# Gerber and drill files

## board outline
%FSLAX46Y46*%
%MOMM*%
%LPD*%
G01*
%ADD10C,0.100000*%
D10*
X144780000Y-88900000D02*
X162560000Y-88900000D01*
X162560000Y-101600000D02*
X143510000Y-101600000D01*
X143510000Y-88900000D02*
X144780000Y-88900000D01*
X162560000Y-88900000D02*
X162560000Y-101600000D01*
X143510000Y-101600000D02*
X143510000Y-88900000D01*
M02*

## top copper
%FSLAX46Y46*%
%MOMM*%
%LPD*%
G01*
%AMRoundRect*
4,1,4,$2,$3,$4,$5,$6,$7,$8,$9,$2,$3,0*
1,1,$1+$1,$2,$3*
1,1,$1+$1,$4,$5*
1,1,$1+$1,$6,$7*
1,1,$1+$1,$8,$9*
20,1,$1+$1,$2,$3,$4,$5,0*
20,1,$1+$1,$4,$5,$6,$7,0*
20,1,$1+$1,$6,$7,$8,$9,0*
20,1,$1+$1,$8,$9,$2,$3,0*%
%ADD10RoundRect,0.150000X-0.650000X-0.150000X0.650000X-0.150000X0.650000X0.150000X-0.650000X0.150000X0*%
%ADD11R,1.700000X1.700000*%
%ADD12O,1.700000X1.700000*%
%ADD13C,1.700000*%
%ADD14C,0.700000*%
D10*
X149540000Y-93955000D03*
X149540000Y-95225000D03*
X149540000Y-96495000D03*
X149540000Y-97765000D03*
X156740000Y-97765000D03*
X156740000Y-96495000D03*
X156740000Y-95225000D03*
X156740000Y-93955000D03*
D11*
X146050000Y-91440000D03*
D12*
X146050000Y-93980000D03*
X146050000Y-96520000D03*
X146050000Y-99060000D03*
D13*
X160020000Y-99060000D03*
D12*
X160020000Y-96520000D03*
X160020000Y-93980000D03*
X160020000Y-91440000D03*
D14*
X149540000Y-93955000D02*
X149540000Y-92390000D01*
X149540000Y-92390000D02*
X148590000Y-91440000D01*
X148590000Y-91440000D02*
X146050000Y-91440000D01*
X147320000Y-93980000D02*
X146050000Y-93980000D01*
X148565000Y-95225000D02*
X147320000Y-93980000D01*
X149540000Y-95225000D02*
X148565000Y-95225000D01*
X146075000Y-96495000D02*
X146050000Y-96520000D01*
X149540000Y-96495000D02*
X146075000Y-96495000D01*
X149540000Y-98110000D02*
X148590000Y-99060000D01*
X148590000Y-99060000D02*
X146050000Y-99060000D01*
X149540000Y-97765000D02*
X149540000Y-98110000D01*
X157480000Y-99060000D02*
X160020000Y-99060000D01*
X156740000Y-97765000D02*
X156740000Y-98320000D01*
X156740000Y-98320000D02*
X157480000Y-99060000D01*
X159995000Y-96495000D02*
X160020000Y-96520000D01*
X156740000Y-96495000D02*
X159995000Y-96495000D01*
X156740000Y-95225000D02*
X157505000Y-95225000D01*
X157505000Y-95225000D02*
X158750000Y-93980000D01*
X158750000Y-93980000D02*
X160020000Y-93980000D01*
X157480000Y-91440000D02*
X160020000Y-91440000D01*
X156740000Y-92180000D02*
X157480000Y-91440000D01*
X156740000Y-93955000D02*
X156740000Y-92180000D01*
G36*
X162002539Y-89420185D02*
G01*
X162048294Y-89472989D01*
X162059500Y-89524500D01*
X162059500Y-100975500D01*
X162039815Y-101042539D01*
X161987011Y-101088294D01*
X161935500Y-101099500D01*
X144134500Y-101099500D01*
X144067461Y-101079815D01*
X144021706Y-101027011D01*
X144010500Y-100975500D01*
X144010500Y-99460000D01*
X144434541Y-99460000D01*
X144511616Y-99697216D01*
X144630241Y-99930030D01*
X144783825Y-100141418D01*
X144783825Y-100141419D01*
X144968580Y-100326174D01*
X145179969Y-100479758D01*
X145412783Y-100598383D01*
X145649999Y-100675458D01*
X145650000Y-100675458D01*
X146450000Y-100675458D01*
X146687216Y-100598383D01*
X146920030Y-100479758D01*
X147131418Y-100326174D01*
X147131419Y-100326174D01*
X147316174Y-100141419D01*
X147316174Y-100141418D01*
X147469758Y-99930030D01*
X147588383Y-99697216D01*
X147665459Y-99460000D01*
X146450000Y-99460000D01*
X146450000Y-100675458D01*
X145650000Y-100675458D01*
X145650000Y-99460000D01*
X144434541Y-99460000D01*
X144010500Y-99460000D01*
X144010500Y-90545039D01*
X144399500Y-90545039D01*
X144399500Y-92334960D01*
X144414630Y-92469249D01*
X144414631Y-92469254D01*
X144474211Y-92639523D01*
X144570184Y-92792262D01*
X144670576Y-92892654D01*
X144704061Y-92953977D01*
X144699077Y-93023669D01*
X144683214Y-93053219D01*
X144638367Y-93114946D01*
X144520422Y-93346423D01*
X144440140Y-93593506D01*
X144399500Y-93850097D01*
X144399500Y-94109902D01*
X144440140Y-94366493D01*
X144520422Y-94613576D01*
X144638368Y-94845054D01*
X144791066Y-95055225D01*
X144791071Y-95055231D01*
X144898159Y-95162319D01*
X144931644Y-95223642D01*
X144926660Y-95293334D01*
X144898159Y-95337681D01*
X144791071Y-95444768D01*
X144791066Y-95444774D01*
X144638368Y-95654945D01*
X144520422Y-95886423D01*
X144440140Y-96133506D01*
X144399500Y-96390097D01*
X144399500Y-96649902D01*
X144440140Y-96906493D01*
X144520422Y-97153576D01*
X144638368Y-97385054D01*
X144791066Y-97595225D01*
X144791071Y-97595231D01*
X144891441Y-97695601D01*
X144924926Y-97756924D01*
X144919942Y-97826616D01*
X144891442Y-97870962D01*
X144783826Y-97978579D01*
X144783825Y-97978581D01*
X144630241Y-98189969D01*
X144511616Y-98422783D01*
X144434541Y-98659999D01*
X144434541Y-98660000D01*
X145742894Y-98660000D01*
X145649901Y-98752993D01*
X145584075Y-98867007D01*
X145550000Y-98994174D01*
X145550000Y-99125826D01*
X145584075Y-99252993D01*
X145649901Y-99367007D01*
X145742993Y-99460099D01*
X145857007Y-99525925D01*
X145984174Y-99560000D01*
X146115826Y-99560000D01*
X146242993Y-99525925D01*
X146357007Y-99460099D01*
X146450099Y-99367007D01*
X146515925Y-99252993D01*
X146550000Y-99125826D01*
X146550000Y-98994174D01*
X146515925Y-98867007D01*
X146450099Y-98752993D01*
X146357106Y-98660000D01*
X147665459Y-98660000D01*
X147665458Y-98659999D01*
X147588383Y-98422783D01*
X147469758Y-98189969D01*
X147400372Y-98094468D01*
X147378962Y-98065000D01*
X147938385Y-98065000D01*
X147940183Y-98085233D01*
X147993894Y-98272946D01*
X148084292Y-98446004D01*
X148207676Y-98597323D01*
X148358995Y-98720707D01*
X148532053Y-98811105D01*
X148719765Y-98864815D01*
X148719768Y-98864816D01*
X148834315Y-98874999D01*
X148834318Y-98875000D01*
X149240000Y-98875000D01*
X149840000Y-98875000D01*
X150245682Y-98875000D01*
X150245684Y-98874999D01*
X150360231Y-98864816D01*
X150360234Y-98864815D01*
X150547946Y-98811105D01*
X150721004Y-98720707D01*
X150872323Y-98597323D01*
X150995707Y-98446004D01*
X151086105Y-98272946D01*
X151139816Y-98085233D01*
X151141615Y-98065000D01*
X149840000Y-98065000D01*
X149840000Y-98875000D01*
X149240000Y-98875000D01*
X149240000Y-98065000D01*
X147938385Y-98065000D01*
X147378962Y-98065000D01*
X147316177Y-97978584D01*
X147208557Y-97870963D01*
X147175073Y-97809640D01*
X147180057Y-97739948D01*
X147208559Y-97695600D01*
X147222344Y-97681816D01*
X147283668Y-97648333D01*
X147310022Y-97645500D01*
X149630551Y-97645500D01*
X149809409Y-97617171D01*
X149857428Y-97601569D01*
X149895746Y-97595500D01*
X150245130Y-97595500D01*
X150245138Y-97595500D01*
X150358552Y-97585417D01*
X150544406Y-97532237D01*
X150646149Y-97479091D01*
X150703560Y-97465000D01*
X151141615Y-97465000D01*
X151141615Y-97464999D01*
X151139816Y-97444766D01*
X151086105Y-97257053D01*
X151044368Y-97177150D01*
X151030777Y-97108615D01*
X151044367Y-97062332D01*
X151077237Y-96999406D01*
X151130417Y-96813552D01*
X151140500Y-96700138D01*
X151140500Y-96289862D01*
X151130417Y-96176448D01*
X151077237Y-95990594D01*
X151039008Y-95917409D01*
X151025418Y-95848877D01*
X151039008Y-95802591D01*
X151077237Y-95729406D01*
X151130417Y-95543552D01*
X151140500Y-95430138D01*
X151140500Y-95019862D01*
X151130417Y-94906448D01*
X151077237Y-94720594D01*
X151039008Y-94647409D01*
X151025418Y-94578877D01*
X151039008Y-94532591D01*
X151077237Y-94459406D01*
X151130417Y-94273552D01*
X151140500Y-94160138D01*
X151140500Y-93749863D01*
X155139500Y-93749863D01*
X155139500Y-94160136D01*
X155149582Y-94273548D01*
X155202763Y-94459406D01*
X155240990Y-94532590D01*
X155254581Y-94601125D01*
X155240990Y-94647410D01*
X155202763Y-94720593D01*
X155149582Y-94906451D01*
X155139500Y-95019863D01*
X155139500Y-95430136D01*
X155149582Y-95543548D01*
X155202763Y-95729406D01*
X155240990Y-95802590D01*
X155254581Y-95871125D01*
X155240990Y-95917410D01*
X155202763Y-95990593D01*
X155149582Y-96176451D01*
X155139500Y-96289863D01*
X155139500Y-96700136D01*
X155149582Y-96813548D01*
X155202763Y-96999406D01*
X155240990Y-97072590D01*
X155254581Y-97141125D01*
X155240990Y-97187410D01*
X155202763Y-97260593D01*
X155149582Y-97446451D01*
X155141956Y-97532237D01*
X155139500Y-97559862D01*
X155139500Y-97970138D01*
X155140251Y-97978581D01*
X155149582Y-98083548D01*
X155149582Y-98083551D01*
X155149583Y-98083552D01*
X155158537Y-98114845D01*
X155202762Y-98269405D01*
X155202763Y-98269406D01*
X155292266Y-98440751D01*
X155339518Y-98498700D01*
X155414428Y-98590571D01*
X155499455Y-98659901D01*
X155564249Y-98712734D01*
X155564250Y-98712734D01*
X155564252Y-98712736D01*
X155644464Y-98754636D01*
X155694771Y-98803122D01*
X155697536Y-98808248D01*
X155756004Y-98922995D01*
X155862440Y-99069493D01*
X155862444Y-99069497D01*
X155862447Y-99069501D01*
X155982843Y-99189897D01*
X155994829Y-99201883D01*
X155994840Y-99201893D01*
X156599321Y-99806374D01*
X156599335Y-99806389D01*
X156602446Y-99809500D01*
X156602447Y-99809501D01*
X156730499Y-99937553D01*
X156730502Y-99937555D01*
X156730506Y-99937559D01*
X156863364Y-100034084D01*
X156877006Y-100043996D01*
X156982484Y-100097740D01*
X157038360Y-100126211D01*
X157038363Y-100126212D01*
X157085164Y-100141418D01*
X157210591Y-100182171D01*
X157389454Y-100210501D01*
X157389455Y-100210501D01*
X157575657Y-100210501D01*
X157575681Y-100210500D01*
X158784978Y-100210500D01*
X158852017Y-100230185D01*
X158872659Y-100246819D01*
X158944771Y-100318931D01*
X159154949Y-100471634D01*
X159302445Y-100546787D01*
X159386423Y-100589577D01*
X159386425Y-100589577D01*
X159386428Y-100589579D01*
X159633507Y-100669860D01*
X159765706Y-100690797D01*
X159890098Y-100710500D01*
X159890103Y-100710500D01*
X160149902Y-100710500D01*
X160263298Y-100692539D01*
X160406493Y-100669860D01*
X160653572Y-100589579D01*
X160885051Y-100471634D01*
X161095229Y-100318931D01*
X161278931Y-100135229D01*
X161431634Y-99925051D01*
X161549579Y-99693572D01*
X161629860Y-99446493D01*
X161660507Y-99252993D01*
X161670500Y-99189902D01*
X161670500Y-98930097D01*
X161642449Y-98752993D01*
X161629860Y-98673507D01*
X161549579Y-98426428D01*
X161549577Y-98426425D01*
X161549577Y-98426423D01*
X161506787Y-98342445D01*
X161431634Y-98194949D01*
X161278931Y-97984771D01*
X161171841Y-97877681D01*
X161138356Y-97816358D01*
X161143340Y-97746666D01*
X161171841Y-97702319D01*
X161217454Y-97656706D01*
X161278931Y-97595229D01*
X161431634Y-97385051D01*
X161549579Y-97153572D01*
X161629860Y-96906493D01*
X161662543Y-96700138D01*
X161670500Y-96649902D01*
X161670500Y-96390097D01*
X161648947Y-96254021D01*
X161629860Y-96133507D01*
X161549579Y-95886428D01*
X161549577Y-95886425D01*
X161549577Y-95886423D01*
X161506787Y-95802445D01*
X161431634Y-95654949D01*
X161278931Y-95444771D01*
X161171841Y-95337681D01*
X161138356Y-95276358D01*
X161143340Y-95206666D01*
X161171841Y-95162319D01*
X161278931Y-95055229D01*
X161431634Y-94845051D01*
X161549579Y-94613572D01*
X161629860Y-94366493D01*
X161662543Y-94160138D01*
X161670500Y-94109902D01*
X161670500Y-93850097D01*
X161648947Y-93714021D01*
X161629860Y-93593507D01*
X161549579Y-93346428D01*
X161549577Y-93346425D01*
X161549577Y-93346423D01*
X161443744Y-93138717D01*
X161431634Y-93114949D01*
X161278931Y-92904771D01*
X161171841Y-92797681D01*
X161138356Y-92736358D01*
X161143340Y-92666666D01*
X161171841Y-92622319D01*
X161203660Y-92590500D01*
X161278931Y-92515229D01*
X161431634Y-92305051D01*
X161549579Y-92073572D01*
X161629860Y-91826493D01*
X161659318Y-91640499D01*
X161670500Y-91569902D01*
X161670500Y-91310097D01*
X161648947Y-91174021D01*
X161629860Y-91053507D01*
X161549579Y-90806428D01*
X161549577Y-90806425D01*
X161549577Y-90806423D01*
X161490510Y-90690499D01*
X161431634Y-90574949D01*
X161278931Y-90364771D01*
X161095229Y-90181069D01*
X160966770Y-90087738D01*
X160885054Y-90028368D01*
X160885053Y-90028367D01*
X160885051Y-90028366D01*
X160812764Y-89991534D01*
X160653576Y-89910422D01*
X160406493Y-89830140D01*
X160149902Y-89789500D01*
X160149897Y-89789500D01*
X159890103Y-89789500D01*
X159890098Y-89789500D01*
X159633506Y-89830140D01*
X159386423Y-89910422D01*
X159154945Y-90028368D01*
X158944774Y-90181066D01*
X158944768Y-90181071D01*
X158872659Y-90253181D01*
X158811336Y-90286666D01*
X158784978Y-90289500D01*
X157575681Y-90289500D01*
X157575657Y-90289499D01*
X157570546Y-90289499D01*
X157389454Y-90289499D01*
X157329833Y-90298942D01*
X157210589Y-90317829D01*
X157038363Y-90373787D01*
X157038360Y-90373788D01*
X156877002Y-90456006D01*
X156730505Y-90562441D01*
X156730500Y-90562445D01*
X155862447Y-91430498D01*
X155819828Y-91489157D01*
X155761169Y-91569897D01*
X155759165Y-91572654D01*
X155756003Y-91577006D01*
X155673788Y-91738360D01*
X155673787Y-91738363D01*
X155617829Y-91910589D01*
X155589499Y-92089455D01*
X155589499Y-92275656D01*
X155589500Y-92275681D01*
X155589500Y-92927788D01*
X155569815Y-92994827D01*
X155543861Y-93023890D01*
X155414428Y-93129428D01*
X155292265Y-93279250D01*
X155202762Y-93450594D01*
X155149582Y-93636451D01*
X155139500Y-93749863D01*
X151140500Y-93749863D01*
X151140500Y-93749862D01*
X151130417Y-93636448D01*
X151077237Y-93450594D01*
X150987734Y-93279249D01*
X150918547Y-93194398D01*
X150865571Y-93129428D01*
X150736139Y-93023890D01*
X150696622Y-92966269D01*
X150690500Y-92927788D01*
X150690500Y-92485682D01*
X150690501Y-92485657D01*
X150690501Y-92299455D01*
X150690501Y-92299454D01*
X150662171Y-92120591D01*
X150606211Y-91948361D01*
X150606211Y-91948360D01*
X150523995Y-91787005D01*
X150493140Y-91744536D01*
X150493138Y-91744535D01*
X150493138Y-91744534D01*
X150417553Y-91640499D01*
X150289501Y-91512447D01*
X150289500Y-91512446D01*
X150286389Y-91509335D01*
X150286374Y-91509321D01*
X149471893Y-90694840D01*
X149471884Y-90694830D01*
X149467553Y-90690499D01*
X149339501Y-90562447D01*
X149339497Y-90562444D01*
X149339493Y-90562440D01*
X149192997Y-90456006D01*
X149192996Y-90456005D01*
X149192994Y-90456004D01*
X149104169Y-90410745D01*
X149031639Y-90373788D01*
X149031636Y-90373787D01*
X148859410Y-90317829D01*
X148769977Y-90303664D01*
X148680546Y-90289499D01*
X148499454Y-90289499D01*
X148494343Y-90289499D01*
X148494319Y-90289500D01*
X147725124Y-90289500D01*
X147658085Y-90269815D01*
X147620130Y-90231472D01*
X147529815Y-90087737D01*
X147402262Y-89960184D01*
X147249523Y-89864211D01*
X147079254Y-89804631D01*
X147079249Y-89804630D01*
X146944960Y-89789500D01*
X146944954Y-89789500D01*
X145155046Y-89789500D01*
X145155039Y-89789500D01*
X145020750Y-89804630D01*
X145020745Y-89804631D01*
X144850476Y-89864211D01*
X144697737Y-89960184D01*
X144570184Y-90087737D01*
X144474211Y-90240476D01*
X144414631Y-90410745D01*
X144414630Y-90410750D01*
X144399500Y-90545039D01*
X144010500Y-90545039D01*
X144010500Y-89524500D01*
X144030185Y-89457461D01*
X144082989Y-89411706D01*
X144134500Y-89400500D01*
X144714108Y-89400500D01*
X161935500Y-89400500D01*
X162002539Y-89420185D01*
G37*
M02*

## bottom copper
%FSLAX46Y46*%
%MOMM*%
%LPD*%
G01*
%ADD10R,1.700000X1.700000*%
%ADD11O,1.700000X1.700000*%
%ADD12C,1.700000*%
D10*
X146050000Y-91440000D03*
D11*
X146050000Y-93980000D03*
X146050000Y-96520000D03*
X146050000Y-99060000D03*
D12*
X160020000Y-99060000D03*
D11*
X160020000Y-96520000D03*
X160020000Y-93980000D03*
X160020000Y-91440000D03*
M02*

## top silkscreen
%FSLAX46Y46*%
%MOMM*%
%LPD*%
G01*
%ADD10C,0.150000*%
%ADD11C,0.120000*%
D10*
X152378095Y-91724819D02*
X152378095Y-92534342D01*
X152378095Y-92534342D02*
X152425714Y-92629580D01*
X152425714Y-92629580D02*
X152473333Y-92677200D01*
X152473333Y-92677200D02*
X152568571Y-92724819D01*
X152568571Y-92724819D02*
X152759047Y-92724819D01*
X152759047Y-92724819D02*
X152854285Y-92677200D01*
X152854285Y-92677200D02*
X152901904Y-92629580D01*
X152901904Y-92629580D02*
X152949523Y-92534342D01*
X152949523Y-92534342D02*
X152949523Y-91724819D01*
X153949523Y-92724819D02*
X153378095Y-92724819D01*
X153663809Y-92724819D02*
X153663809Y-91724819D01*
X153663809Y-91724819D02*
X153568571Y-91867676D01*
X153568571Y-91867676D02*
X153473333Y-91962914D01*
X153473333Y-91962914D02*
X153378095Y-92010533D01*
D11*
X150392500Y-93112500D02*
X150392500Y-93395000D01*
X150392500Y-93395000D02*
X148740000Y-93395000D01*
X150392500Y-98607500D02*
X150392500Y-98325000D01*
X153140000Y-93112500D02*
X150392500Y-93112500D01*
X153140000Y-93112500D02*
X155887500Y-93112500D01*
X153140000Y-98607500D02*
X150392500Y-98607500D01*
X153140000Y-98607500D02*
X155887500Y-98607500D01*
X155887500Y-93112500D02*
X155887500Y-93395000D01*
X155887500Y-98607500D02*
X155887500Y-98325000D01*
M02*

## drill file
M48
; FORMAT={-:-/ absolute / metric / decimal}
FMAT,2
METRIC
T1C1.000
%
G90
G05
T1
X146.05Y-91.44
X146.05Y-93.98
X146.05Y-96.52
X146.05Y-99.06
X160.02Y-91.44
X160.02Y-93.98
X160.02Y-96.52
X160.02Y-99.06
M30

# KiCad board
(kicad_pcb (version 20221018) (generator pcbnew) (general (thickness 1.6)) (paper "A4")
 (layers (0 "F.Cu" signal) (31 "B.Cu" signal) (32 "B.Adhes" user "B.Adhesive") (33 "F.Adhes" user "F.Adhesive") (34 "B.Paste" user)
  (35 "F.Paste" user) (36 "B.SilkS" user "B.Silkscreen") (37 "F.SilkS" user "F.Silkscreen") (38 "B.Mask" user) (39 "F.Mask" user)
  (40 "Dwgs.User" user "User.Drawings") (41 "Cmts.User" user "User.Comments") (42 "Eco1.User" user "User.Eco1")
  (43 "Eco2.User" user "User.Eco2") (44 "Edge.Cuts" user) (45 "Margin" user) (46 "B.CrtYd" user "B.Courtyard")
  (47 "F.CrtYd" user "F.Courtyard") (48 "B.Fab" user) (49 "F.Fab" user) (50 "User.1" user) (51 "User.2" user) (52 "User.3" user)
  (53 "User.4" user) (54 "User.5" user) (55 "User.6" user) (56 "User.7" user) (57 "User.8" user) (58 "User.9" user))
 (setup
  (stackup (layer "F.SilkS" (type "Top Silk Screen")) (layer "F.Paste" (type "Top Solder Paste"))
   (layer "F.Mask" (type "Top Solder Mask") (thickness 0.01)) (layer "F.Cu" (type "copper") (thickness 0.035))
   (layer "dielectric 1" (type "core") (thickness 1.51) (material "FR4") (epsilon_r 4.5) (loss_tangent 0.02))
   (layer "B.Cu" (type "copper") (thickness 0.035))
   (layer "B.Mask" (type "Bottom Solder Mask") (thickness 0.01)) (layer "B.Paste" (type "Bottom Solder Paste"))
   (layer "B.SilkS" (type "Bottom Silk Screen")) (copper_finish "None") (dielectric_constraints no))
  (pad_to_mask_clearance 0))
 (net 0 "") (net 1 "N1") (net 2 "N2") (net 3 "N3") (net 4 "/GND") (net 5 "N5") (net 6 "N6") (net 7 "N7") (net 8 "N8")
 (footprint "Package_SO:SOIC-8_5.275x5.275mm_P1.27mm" (layer "F.Cu") (at 153.14 95.86)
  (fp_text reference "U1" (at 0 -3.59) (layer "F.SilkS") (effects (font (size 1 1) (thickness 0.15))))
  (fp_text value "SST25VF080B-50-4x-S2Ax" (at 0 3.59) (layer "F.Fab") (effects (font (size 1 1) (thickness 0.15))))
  (fp_line (start -2.7475 -2.7475) (end -2.7475 -2.465) (stroke (width 0.12) (type solid)) (layer "F.SilkS"))
  (fp_line (start -2.7475 -2.465) (end -4.4 -2.465) (stroke (width 0.12) (type solid)) (layer "F.SilkS"))
  (fp_line (start -2.7475 2.7475) (end -2.7475 2.465) (stroke (width 0.12) (type solid)) (layer "F.SilkS"))
  (fp_line (start 0 -2.7475) (end -2.7475 -2.7475) (stroke (width 0.12) (type solid)) (layer "F.SilkS"))
  (fp_line (start 0 -2.7475) (end 2.7475 -2.7475) (stroke (width 0.12) (type solid)) (layer "F.SilkS"))
  (fp_line (start 0 2.7475) (end -2.7475 2.7475) (stroke (width 0.12) (type solid)) (layer "F.SilkS"))
  (fp_line (start 0 2.7475) (end 2.7475 2.7475) (stroke (width 0.12) (type solid)) (layer "F.SilkS"))
  (fp_line (start 2.7475 -2.7475) (end 2.7475 -2.465) (stroke (width 0.12) (type solid)) (layer "F.SilkS"))
  (fp_line (start 2.7475 2.7475) (end 2.7475 2.465) (stroke (width 0.12) (type solid)) (layer "F.SilkS"))
  (pad "1" smd roundrect (at -3.6 -1.905) (size 1.6 0.6) (layers "F.Cu" "F.Paste" "F.Mask") (roundrect_rratio 0.25) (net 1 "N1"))
  (pad "2" smd roundrect (at -3.6 -0.635) (size 1.6 0.6) (layers "F.Cu" "F.Paste" "F.Mask") (roundrect_rratio 0.25) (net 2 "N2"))
  (pad "3" smd roundrect (at -3.6 0.635) (size 1.6 0.6) (layers "F.Cu" "F.Paste" "F.Mask") (roundrect_rratio 0.25) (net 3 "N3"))
  (pad "4" smd roundrect (at -3.6 1.905) (size 1.6 0.6) (layers "F.Cu" "F.Paste" "F.Mask") (roundrect_rratio 0.25) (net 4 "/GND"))
  (pad "5" smd roundrect (at 3.6 1.905) (size 1.6 0.6) (layers "F.Cu" "F.Paste" "F.Mask") (roundrect_rratio 0.25) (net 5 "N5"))
  (pad "6" smd roundrect (at 3.6 0.635) (size 1.6 0.6) (layers "F.Cu" "F.Paste" "F.Mask") (roundrect_rratio 0.25) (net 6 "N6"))
  (pad "7" smd roundrect (at 3.6 -0.635) (size 1.6 0.6) (layers "F.Cu" "F.Paste" "F.Mask") (roundrect_rratio 0.25) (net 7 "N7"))
  (pad "8" smd roundrect (at 3.6 -1.905) (size 1.6 0.6) (layers "F.Cu" "F.Paste" "F.Mask") (roundrect_rratio 0.25) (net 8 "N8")))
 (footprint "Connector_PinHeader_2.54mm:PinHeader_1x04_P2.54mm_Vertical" (layer "B.Cu") (at 146.05 91.44 180)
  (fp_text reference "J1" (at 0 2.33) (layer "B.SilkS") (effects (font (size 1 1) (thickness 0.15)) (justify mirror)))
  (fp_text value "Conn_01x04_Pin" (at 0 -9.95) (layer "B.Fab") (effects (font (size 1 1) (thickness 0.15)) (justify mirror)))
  (pad "1" thru_hole rect (at 0 0 180) (size 1.7 1.7) (drill 1) (layers "*.Cu" "*.Mask") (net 1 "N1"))
  (pad "2" thru_hole oval (at 0 -2.54 180) (size 1.7 1.7) (drill 1) (layers "*.Cu" "*.Mask") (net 2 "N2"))
  (pad "3" thru_hole oval (at 0 -5.08 180) (size 1.7 1.7) (drill 1) (layers "*.Cu" "*.Mask") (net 3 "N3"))
  (pad "4" thru_hole oval (at 0 -7.62 180) (size 1.7 1.7) (drill 1) (layers "*.Cu" "*.Mask") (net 4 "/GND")))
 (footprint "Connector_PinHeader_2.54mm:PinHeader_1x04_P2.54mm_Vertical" (layer "B.Cu") (at 160.02 99.06)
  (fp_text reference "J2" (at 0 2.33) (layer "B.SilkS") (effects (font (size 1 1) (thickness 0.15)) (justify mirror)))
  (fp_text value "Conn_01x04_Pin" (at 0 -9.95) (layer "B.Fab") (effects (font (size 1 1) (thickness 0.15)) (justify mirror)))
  (pad "5" thru_hole circle (at 0 0) (size 1.7 1.7) (drill 1) (layers "*.Cu" "*.Mask") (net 5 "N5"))
  (pad "6" thru_hole oval (at 0 -2.54) (size 1.7 1.7) (drill 1) (layers "*.Cu" "*.Mask") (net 6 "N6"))
  (pad "7" thru_hole oval (at 0 -5.08) (size 1.7 1.7) (drill 1) (layers "*.Cu" "*.Mask") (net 7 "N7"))
  (pad "8" thru_hole oval (at 0 -7.62) (size 1.7 1.7) (drill 1) (layers "*.Cu" "*.Mask") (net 8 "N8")))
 (gr_line (start 144.78 88.9) (end 162.56 88.9) (stroke (width 0.1) (type default)) (layer "Edge.Cuts"))
 (gr_line (start 162.56 101.6) (end 143.51 101.6) (stroke (width 0.1) (type default)) (layer "Edge.Cuts"))
 (gr_line (start 143.51 88.9) (end 144.78 88.9) (stroke (width 0.1) (type default)) (layer "Edge.Cuts"))
 (gr_line (start 162.56 88.9) (end 162.56 101.6) (stroke (width 0.1) (type default)) (layer "Edge.Cuts"))
 (gr_line (start 143.51 101.6) (end 143.51 88.9) (stroke (width 0.1) (type default)) (layer "Edge.Cuts"))
 (segment (start 149.54 93.955) (end 149.54 92.39) (width 0.7) (layer "F.Cu") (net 1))
 (segment (start 149.54 92.39) (end 148.59 91.44) (width 0.7) (layer "F.Cu") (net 1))
 (segment (start 148.59 91.44) (end 146.05 91.44) (width 0.7) (layer "F.Cu") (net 1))
 (segment (start 147.32 93.98) (end 146.05 93.98) (width 0.7) (layer "F.Cu") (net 2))
 (segment (start 148.565 95.225) (end 147.32 93.98) (width 0.7) (layer "F.Cu") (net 2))
 (segment (start 149.54 95.225) (end 148.565 95.225) (width 0.7) (layer "F.Cu") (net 2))
 (segment (start 146.075 96.495) (end 146.05 96.52) (width 0.7) (layer "F.Cu") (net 3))
 (segment (start 149.54 96.495) (end 146.075 96.495) (width 0.7) (layer "F.Cu") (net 3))
 (segment (start 149.54 98.11) (end 148.59 99.06) (width 0.7) (layer "F.Cu") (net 4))
 (segment (start 148.59 99.06) (end 146.05 99.06) (width 0.7) (layer "F.Cu") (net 4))
 (segment (start 149.54 97.765) (end 149.54 98.11) (width 0.7) (layer "F.Cu") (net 4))
 (segment (start 157.48 99.06) (end 160.02 99.06) (width 0.7) (layer "F.Cu") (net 5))
 (segment (start 156.74 97.765) (end 156.74 98.32) (width 0.7) (layer "F.Cu") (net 5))
 (segment (start 156.74 98.32) (end 157.48 99.06) (width 0.7) (layer "F.Cu") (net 5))
 (segment (start 159.995 96.495) (end 160.02 96.52) (width 0.7) (layer "F.Cu") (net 6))
 (segment (start 156.74 96.495) (end 159.995 96.495) (width 0.7) (layer "F.Cu") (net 6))
 (segment (start 156.74 95.225) (end 157.505 95.225) (width 0.7) (layer "F.Cu") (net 7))
 (segment (start 157.505 95.225) (end 158.75 93.98) (width 0.7) (layer "F.Cu") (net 7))
 (segment (start 158.75 93.98) (end 160.02 93.98) (width 0.7) (layer "F.Cu") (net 7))
 (segment (start 157.48 91.44) (end 160.02 91.44) (width 0.7) (layer "F.Cu") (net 8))
 (segment (start 156.74 92.18) (end 157.48 91.44) (width 0.7) (layer "F.Cu") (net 8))
 (segment (start 156.74 93.955) (end 156.74 92.18) (width 0.7) (layer "F.Cu") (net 8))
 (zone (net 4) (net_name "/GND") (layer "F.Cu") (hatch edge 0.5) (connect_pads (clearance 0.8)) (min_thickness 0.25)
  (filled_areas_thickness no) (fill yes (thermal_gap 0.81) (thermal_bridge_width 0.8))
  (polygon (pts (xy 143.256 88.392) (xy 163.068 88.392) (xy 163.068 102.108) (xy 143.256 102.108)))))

